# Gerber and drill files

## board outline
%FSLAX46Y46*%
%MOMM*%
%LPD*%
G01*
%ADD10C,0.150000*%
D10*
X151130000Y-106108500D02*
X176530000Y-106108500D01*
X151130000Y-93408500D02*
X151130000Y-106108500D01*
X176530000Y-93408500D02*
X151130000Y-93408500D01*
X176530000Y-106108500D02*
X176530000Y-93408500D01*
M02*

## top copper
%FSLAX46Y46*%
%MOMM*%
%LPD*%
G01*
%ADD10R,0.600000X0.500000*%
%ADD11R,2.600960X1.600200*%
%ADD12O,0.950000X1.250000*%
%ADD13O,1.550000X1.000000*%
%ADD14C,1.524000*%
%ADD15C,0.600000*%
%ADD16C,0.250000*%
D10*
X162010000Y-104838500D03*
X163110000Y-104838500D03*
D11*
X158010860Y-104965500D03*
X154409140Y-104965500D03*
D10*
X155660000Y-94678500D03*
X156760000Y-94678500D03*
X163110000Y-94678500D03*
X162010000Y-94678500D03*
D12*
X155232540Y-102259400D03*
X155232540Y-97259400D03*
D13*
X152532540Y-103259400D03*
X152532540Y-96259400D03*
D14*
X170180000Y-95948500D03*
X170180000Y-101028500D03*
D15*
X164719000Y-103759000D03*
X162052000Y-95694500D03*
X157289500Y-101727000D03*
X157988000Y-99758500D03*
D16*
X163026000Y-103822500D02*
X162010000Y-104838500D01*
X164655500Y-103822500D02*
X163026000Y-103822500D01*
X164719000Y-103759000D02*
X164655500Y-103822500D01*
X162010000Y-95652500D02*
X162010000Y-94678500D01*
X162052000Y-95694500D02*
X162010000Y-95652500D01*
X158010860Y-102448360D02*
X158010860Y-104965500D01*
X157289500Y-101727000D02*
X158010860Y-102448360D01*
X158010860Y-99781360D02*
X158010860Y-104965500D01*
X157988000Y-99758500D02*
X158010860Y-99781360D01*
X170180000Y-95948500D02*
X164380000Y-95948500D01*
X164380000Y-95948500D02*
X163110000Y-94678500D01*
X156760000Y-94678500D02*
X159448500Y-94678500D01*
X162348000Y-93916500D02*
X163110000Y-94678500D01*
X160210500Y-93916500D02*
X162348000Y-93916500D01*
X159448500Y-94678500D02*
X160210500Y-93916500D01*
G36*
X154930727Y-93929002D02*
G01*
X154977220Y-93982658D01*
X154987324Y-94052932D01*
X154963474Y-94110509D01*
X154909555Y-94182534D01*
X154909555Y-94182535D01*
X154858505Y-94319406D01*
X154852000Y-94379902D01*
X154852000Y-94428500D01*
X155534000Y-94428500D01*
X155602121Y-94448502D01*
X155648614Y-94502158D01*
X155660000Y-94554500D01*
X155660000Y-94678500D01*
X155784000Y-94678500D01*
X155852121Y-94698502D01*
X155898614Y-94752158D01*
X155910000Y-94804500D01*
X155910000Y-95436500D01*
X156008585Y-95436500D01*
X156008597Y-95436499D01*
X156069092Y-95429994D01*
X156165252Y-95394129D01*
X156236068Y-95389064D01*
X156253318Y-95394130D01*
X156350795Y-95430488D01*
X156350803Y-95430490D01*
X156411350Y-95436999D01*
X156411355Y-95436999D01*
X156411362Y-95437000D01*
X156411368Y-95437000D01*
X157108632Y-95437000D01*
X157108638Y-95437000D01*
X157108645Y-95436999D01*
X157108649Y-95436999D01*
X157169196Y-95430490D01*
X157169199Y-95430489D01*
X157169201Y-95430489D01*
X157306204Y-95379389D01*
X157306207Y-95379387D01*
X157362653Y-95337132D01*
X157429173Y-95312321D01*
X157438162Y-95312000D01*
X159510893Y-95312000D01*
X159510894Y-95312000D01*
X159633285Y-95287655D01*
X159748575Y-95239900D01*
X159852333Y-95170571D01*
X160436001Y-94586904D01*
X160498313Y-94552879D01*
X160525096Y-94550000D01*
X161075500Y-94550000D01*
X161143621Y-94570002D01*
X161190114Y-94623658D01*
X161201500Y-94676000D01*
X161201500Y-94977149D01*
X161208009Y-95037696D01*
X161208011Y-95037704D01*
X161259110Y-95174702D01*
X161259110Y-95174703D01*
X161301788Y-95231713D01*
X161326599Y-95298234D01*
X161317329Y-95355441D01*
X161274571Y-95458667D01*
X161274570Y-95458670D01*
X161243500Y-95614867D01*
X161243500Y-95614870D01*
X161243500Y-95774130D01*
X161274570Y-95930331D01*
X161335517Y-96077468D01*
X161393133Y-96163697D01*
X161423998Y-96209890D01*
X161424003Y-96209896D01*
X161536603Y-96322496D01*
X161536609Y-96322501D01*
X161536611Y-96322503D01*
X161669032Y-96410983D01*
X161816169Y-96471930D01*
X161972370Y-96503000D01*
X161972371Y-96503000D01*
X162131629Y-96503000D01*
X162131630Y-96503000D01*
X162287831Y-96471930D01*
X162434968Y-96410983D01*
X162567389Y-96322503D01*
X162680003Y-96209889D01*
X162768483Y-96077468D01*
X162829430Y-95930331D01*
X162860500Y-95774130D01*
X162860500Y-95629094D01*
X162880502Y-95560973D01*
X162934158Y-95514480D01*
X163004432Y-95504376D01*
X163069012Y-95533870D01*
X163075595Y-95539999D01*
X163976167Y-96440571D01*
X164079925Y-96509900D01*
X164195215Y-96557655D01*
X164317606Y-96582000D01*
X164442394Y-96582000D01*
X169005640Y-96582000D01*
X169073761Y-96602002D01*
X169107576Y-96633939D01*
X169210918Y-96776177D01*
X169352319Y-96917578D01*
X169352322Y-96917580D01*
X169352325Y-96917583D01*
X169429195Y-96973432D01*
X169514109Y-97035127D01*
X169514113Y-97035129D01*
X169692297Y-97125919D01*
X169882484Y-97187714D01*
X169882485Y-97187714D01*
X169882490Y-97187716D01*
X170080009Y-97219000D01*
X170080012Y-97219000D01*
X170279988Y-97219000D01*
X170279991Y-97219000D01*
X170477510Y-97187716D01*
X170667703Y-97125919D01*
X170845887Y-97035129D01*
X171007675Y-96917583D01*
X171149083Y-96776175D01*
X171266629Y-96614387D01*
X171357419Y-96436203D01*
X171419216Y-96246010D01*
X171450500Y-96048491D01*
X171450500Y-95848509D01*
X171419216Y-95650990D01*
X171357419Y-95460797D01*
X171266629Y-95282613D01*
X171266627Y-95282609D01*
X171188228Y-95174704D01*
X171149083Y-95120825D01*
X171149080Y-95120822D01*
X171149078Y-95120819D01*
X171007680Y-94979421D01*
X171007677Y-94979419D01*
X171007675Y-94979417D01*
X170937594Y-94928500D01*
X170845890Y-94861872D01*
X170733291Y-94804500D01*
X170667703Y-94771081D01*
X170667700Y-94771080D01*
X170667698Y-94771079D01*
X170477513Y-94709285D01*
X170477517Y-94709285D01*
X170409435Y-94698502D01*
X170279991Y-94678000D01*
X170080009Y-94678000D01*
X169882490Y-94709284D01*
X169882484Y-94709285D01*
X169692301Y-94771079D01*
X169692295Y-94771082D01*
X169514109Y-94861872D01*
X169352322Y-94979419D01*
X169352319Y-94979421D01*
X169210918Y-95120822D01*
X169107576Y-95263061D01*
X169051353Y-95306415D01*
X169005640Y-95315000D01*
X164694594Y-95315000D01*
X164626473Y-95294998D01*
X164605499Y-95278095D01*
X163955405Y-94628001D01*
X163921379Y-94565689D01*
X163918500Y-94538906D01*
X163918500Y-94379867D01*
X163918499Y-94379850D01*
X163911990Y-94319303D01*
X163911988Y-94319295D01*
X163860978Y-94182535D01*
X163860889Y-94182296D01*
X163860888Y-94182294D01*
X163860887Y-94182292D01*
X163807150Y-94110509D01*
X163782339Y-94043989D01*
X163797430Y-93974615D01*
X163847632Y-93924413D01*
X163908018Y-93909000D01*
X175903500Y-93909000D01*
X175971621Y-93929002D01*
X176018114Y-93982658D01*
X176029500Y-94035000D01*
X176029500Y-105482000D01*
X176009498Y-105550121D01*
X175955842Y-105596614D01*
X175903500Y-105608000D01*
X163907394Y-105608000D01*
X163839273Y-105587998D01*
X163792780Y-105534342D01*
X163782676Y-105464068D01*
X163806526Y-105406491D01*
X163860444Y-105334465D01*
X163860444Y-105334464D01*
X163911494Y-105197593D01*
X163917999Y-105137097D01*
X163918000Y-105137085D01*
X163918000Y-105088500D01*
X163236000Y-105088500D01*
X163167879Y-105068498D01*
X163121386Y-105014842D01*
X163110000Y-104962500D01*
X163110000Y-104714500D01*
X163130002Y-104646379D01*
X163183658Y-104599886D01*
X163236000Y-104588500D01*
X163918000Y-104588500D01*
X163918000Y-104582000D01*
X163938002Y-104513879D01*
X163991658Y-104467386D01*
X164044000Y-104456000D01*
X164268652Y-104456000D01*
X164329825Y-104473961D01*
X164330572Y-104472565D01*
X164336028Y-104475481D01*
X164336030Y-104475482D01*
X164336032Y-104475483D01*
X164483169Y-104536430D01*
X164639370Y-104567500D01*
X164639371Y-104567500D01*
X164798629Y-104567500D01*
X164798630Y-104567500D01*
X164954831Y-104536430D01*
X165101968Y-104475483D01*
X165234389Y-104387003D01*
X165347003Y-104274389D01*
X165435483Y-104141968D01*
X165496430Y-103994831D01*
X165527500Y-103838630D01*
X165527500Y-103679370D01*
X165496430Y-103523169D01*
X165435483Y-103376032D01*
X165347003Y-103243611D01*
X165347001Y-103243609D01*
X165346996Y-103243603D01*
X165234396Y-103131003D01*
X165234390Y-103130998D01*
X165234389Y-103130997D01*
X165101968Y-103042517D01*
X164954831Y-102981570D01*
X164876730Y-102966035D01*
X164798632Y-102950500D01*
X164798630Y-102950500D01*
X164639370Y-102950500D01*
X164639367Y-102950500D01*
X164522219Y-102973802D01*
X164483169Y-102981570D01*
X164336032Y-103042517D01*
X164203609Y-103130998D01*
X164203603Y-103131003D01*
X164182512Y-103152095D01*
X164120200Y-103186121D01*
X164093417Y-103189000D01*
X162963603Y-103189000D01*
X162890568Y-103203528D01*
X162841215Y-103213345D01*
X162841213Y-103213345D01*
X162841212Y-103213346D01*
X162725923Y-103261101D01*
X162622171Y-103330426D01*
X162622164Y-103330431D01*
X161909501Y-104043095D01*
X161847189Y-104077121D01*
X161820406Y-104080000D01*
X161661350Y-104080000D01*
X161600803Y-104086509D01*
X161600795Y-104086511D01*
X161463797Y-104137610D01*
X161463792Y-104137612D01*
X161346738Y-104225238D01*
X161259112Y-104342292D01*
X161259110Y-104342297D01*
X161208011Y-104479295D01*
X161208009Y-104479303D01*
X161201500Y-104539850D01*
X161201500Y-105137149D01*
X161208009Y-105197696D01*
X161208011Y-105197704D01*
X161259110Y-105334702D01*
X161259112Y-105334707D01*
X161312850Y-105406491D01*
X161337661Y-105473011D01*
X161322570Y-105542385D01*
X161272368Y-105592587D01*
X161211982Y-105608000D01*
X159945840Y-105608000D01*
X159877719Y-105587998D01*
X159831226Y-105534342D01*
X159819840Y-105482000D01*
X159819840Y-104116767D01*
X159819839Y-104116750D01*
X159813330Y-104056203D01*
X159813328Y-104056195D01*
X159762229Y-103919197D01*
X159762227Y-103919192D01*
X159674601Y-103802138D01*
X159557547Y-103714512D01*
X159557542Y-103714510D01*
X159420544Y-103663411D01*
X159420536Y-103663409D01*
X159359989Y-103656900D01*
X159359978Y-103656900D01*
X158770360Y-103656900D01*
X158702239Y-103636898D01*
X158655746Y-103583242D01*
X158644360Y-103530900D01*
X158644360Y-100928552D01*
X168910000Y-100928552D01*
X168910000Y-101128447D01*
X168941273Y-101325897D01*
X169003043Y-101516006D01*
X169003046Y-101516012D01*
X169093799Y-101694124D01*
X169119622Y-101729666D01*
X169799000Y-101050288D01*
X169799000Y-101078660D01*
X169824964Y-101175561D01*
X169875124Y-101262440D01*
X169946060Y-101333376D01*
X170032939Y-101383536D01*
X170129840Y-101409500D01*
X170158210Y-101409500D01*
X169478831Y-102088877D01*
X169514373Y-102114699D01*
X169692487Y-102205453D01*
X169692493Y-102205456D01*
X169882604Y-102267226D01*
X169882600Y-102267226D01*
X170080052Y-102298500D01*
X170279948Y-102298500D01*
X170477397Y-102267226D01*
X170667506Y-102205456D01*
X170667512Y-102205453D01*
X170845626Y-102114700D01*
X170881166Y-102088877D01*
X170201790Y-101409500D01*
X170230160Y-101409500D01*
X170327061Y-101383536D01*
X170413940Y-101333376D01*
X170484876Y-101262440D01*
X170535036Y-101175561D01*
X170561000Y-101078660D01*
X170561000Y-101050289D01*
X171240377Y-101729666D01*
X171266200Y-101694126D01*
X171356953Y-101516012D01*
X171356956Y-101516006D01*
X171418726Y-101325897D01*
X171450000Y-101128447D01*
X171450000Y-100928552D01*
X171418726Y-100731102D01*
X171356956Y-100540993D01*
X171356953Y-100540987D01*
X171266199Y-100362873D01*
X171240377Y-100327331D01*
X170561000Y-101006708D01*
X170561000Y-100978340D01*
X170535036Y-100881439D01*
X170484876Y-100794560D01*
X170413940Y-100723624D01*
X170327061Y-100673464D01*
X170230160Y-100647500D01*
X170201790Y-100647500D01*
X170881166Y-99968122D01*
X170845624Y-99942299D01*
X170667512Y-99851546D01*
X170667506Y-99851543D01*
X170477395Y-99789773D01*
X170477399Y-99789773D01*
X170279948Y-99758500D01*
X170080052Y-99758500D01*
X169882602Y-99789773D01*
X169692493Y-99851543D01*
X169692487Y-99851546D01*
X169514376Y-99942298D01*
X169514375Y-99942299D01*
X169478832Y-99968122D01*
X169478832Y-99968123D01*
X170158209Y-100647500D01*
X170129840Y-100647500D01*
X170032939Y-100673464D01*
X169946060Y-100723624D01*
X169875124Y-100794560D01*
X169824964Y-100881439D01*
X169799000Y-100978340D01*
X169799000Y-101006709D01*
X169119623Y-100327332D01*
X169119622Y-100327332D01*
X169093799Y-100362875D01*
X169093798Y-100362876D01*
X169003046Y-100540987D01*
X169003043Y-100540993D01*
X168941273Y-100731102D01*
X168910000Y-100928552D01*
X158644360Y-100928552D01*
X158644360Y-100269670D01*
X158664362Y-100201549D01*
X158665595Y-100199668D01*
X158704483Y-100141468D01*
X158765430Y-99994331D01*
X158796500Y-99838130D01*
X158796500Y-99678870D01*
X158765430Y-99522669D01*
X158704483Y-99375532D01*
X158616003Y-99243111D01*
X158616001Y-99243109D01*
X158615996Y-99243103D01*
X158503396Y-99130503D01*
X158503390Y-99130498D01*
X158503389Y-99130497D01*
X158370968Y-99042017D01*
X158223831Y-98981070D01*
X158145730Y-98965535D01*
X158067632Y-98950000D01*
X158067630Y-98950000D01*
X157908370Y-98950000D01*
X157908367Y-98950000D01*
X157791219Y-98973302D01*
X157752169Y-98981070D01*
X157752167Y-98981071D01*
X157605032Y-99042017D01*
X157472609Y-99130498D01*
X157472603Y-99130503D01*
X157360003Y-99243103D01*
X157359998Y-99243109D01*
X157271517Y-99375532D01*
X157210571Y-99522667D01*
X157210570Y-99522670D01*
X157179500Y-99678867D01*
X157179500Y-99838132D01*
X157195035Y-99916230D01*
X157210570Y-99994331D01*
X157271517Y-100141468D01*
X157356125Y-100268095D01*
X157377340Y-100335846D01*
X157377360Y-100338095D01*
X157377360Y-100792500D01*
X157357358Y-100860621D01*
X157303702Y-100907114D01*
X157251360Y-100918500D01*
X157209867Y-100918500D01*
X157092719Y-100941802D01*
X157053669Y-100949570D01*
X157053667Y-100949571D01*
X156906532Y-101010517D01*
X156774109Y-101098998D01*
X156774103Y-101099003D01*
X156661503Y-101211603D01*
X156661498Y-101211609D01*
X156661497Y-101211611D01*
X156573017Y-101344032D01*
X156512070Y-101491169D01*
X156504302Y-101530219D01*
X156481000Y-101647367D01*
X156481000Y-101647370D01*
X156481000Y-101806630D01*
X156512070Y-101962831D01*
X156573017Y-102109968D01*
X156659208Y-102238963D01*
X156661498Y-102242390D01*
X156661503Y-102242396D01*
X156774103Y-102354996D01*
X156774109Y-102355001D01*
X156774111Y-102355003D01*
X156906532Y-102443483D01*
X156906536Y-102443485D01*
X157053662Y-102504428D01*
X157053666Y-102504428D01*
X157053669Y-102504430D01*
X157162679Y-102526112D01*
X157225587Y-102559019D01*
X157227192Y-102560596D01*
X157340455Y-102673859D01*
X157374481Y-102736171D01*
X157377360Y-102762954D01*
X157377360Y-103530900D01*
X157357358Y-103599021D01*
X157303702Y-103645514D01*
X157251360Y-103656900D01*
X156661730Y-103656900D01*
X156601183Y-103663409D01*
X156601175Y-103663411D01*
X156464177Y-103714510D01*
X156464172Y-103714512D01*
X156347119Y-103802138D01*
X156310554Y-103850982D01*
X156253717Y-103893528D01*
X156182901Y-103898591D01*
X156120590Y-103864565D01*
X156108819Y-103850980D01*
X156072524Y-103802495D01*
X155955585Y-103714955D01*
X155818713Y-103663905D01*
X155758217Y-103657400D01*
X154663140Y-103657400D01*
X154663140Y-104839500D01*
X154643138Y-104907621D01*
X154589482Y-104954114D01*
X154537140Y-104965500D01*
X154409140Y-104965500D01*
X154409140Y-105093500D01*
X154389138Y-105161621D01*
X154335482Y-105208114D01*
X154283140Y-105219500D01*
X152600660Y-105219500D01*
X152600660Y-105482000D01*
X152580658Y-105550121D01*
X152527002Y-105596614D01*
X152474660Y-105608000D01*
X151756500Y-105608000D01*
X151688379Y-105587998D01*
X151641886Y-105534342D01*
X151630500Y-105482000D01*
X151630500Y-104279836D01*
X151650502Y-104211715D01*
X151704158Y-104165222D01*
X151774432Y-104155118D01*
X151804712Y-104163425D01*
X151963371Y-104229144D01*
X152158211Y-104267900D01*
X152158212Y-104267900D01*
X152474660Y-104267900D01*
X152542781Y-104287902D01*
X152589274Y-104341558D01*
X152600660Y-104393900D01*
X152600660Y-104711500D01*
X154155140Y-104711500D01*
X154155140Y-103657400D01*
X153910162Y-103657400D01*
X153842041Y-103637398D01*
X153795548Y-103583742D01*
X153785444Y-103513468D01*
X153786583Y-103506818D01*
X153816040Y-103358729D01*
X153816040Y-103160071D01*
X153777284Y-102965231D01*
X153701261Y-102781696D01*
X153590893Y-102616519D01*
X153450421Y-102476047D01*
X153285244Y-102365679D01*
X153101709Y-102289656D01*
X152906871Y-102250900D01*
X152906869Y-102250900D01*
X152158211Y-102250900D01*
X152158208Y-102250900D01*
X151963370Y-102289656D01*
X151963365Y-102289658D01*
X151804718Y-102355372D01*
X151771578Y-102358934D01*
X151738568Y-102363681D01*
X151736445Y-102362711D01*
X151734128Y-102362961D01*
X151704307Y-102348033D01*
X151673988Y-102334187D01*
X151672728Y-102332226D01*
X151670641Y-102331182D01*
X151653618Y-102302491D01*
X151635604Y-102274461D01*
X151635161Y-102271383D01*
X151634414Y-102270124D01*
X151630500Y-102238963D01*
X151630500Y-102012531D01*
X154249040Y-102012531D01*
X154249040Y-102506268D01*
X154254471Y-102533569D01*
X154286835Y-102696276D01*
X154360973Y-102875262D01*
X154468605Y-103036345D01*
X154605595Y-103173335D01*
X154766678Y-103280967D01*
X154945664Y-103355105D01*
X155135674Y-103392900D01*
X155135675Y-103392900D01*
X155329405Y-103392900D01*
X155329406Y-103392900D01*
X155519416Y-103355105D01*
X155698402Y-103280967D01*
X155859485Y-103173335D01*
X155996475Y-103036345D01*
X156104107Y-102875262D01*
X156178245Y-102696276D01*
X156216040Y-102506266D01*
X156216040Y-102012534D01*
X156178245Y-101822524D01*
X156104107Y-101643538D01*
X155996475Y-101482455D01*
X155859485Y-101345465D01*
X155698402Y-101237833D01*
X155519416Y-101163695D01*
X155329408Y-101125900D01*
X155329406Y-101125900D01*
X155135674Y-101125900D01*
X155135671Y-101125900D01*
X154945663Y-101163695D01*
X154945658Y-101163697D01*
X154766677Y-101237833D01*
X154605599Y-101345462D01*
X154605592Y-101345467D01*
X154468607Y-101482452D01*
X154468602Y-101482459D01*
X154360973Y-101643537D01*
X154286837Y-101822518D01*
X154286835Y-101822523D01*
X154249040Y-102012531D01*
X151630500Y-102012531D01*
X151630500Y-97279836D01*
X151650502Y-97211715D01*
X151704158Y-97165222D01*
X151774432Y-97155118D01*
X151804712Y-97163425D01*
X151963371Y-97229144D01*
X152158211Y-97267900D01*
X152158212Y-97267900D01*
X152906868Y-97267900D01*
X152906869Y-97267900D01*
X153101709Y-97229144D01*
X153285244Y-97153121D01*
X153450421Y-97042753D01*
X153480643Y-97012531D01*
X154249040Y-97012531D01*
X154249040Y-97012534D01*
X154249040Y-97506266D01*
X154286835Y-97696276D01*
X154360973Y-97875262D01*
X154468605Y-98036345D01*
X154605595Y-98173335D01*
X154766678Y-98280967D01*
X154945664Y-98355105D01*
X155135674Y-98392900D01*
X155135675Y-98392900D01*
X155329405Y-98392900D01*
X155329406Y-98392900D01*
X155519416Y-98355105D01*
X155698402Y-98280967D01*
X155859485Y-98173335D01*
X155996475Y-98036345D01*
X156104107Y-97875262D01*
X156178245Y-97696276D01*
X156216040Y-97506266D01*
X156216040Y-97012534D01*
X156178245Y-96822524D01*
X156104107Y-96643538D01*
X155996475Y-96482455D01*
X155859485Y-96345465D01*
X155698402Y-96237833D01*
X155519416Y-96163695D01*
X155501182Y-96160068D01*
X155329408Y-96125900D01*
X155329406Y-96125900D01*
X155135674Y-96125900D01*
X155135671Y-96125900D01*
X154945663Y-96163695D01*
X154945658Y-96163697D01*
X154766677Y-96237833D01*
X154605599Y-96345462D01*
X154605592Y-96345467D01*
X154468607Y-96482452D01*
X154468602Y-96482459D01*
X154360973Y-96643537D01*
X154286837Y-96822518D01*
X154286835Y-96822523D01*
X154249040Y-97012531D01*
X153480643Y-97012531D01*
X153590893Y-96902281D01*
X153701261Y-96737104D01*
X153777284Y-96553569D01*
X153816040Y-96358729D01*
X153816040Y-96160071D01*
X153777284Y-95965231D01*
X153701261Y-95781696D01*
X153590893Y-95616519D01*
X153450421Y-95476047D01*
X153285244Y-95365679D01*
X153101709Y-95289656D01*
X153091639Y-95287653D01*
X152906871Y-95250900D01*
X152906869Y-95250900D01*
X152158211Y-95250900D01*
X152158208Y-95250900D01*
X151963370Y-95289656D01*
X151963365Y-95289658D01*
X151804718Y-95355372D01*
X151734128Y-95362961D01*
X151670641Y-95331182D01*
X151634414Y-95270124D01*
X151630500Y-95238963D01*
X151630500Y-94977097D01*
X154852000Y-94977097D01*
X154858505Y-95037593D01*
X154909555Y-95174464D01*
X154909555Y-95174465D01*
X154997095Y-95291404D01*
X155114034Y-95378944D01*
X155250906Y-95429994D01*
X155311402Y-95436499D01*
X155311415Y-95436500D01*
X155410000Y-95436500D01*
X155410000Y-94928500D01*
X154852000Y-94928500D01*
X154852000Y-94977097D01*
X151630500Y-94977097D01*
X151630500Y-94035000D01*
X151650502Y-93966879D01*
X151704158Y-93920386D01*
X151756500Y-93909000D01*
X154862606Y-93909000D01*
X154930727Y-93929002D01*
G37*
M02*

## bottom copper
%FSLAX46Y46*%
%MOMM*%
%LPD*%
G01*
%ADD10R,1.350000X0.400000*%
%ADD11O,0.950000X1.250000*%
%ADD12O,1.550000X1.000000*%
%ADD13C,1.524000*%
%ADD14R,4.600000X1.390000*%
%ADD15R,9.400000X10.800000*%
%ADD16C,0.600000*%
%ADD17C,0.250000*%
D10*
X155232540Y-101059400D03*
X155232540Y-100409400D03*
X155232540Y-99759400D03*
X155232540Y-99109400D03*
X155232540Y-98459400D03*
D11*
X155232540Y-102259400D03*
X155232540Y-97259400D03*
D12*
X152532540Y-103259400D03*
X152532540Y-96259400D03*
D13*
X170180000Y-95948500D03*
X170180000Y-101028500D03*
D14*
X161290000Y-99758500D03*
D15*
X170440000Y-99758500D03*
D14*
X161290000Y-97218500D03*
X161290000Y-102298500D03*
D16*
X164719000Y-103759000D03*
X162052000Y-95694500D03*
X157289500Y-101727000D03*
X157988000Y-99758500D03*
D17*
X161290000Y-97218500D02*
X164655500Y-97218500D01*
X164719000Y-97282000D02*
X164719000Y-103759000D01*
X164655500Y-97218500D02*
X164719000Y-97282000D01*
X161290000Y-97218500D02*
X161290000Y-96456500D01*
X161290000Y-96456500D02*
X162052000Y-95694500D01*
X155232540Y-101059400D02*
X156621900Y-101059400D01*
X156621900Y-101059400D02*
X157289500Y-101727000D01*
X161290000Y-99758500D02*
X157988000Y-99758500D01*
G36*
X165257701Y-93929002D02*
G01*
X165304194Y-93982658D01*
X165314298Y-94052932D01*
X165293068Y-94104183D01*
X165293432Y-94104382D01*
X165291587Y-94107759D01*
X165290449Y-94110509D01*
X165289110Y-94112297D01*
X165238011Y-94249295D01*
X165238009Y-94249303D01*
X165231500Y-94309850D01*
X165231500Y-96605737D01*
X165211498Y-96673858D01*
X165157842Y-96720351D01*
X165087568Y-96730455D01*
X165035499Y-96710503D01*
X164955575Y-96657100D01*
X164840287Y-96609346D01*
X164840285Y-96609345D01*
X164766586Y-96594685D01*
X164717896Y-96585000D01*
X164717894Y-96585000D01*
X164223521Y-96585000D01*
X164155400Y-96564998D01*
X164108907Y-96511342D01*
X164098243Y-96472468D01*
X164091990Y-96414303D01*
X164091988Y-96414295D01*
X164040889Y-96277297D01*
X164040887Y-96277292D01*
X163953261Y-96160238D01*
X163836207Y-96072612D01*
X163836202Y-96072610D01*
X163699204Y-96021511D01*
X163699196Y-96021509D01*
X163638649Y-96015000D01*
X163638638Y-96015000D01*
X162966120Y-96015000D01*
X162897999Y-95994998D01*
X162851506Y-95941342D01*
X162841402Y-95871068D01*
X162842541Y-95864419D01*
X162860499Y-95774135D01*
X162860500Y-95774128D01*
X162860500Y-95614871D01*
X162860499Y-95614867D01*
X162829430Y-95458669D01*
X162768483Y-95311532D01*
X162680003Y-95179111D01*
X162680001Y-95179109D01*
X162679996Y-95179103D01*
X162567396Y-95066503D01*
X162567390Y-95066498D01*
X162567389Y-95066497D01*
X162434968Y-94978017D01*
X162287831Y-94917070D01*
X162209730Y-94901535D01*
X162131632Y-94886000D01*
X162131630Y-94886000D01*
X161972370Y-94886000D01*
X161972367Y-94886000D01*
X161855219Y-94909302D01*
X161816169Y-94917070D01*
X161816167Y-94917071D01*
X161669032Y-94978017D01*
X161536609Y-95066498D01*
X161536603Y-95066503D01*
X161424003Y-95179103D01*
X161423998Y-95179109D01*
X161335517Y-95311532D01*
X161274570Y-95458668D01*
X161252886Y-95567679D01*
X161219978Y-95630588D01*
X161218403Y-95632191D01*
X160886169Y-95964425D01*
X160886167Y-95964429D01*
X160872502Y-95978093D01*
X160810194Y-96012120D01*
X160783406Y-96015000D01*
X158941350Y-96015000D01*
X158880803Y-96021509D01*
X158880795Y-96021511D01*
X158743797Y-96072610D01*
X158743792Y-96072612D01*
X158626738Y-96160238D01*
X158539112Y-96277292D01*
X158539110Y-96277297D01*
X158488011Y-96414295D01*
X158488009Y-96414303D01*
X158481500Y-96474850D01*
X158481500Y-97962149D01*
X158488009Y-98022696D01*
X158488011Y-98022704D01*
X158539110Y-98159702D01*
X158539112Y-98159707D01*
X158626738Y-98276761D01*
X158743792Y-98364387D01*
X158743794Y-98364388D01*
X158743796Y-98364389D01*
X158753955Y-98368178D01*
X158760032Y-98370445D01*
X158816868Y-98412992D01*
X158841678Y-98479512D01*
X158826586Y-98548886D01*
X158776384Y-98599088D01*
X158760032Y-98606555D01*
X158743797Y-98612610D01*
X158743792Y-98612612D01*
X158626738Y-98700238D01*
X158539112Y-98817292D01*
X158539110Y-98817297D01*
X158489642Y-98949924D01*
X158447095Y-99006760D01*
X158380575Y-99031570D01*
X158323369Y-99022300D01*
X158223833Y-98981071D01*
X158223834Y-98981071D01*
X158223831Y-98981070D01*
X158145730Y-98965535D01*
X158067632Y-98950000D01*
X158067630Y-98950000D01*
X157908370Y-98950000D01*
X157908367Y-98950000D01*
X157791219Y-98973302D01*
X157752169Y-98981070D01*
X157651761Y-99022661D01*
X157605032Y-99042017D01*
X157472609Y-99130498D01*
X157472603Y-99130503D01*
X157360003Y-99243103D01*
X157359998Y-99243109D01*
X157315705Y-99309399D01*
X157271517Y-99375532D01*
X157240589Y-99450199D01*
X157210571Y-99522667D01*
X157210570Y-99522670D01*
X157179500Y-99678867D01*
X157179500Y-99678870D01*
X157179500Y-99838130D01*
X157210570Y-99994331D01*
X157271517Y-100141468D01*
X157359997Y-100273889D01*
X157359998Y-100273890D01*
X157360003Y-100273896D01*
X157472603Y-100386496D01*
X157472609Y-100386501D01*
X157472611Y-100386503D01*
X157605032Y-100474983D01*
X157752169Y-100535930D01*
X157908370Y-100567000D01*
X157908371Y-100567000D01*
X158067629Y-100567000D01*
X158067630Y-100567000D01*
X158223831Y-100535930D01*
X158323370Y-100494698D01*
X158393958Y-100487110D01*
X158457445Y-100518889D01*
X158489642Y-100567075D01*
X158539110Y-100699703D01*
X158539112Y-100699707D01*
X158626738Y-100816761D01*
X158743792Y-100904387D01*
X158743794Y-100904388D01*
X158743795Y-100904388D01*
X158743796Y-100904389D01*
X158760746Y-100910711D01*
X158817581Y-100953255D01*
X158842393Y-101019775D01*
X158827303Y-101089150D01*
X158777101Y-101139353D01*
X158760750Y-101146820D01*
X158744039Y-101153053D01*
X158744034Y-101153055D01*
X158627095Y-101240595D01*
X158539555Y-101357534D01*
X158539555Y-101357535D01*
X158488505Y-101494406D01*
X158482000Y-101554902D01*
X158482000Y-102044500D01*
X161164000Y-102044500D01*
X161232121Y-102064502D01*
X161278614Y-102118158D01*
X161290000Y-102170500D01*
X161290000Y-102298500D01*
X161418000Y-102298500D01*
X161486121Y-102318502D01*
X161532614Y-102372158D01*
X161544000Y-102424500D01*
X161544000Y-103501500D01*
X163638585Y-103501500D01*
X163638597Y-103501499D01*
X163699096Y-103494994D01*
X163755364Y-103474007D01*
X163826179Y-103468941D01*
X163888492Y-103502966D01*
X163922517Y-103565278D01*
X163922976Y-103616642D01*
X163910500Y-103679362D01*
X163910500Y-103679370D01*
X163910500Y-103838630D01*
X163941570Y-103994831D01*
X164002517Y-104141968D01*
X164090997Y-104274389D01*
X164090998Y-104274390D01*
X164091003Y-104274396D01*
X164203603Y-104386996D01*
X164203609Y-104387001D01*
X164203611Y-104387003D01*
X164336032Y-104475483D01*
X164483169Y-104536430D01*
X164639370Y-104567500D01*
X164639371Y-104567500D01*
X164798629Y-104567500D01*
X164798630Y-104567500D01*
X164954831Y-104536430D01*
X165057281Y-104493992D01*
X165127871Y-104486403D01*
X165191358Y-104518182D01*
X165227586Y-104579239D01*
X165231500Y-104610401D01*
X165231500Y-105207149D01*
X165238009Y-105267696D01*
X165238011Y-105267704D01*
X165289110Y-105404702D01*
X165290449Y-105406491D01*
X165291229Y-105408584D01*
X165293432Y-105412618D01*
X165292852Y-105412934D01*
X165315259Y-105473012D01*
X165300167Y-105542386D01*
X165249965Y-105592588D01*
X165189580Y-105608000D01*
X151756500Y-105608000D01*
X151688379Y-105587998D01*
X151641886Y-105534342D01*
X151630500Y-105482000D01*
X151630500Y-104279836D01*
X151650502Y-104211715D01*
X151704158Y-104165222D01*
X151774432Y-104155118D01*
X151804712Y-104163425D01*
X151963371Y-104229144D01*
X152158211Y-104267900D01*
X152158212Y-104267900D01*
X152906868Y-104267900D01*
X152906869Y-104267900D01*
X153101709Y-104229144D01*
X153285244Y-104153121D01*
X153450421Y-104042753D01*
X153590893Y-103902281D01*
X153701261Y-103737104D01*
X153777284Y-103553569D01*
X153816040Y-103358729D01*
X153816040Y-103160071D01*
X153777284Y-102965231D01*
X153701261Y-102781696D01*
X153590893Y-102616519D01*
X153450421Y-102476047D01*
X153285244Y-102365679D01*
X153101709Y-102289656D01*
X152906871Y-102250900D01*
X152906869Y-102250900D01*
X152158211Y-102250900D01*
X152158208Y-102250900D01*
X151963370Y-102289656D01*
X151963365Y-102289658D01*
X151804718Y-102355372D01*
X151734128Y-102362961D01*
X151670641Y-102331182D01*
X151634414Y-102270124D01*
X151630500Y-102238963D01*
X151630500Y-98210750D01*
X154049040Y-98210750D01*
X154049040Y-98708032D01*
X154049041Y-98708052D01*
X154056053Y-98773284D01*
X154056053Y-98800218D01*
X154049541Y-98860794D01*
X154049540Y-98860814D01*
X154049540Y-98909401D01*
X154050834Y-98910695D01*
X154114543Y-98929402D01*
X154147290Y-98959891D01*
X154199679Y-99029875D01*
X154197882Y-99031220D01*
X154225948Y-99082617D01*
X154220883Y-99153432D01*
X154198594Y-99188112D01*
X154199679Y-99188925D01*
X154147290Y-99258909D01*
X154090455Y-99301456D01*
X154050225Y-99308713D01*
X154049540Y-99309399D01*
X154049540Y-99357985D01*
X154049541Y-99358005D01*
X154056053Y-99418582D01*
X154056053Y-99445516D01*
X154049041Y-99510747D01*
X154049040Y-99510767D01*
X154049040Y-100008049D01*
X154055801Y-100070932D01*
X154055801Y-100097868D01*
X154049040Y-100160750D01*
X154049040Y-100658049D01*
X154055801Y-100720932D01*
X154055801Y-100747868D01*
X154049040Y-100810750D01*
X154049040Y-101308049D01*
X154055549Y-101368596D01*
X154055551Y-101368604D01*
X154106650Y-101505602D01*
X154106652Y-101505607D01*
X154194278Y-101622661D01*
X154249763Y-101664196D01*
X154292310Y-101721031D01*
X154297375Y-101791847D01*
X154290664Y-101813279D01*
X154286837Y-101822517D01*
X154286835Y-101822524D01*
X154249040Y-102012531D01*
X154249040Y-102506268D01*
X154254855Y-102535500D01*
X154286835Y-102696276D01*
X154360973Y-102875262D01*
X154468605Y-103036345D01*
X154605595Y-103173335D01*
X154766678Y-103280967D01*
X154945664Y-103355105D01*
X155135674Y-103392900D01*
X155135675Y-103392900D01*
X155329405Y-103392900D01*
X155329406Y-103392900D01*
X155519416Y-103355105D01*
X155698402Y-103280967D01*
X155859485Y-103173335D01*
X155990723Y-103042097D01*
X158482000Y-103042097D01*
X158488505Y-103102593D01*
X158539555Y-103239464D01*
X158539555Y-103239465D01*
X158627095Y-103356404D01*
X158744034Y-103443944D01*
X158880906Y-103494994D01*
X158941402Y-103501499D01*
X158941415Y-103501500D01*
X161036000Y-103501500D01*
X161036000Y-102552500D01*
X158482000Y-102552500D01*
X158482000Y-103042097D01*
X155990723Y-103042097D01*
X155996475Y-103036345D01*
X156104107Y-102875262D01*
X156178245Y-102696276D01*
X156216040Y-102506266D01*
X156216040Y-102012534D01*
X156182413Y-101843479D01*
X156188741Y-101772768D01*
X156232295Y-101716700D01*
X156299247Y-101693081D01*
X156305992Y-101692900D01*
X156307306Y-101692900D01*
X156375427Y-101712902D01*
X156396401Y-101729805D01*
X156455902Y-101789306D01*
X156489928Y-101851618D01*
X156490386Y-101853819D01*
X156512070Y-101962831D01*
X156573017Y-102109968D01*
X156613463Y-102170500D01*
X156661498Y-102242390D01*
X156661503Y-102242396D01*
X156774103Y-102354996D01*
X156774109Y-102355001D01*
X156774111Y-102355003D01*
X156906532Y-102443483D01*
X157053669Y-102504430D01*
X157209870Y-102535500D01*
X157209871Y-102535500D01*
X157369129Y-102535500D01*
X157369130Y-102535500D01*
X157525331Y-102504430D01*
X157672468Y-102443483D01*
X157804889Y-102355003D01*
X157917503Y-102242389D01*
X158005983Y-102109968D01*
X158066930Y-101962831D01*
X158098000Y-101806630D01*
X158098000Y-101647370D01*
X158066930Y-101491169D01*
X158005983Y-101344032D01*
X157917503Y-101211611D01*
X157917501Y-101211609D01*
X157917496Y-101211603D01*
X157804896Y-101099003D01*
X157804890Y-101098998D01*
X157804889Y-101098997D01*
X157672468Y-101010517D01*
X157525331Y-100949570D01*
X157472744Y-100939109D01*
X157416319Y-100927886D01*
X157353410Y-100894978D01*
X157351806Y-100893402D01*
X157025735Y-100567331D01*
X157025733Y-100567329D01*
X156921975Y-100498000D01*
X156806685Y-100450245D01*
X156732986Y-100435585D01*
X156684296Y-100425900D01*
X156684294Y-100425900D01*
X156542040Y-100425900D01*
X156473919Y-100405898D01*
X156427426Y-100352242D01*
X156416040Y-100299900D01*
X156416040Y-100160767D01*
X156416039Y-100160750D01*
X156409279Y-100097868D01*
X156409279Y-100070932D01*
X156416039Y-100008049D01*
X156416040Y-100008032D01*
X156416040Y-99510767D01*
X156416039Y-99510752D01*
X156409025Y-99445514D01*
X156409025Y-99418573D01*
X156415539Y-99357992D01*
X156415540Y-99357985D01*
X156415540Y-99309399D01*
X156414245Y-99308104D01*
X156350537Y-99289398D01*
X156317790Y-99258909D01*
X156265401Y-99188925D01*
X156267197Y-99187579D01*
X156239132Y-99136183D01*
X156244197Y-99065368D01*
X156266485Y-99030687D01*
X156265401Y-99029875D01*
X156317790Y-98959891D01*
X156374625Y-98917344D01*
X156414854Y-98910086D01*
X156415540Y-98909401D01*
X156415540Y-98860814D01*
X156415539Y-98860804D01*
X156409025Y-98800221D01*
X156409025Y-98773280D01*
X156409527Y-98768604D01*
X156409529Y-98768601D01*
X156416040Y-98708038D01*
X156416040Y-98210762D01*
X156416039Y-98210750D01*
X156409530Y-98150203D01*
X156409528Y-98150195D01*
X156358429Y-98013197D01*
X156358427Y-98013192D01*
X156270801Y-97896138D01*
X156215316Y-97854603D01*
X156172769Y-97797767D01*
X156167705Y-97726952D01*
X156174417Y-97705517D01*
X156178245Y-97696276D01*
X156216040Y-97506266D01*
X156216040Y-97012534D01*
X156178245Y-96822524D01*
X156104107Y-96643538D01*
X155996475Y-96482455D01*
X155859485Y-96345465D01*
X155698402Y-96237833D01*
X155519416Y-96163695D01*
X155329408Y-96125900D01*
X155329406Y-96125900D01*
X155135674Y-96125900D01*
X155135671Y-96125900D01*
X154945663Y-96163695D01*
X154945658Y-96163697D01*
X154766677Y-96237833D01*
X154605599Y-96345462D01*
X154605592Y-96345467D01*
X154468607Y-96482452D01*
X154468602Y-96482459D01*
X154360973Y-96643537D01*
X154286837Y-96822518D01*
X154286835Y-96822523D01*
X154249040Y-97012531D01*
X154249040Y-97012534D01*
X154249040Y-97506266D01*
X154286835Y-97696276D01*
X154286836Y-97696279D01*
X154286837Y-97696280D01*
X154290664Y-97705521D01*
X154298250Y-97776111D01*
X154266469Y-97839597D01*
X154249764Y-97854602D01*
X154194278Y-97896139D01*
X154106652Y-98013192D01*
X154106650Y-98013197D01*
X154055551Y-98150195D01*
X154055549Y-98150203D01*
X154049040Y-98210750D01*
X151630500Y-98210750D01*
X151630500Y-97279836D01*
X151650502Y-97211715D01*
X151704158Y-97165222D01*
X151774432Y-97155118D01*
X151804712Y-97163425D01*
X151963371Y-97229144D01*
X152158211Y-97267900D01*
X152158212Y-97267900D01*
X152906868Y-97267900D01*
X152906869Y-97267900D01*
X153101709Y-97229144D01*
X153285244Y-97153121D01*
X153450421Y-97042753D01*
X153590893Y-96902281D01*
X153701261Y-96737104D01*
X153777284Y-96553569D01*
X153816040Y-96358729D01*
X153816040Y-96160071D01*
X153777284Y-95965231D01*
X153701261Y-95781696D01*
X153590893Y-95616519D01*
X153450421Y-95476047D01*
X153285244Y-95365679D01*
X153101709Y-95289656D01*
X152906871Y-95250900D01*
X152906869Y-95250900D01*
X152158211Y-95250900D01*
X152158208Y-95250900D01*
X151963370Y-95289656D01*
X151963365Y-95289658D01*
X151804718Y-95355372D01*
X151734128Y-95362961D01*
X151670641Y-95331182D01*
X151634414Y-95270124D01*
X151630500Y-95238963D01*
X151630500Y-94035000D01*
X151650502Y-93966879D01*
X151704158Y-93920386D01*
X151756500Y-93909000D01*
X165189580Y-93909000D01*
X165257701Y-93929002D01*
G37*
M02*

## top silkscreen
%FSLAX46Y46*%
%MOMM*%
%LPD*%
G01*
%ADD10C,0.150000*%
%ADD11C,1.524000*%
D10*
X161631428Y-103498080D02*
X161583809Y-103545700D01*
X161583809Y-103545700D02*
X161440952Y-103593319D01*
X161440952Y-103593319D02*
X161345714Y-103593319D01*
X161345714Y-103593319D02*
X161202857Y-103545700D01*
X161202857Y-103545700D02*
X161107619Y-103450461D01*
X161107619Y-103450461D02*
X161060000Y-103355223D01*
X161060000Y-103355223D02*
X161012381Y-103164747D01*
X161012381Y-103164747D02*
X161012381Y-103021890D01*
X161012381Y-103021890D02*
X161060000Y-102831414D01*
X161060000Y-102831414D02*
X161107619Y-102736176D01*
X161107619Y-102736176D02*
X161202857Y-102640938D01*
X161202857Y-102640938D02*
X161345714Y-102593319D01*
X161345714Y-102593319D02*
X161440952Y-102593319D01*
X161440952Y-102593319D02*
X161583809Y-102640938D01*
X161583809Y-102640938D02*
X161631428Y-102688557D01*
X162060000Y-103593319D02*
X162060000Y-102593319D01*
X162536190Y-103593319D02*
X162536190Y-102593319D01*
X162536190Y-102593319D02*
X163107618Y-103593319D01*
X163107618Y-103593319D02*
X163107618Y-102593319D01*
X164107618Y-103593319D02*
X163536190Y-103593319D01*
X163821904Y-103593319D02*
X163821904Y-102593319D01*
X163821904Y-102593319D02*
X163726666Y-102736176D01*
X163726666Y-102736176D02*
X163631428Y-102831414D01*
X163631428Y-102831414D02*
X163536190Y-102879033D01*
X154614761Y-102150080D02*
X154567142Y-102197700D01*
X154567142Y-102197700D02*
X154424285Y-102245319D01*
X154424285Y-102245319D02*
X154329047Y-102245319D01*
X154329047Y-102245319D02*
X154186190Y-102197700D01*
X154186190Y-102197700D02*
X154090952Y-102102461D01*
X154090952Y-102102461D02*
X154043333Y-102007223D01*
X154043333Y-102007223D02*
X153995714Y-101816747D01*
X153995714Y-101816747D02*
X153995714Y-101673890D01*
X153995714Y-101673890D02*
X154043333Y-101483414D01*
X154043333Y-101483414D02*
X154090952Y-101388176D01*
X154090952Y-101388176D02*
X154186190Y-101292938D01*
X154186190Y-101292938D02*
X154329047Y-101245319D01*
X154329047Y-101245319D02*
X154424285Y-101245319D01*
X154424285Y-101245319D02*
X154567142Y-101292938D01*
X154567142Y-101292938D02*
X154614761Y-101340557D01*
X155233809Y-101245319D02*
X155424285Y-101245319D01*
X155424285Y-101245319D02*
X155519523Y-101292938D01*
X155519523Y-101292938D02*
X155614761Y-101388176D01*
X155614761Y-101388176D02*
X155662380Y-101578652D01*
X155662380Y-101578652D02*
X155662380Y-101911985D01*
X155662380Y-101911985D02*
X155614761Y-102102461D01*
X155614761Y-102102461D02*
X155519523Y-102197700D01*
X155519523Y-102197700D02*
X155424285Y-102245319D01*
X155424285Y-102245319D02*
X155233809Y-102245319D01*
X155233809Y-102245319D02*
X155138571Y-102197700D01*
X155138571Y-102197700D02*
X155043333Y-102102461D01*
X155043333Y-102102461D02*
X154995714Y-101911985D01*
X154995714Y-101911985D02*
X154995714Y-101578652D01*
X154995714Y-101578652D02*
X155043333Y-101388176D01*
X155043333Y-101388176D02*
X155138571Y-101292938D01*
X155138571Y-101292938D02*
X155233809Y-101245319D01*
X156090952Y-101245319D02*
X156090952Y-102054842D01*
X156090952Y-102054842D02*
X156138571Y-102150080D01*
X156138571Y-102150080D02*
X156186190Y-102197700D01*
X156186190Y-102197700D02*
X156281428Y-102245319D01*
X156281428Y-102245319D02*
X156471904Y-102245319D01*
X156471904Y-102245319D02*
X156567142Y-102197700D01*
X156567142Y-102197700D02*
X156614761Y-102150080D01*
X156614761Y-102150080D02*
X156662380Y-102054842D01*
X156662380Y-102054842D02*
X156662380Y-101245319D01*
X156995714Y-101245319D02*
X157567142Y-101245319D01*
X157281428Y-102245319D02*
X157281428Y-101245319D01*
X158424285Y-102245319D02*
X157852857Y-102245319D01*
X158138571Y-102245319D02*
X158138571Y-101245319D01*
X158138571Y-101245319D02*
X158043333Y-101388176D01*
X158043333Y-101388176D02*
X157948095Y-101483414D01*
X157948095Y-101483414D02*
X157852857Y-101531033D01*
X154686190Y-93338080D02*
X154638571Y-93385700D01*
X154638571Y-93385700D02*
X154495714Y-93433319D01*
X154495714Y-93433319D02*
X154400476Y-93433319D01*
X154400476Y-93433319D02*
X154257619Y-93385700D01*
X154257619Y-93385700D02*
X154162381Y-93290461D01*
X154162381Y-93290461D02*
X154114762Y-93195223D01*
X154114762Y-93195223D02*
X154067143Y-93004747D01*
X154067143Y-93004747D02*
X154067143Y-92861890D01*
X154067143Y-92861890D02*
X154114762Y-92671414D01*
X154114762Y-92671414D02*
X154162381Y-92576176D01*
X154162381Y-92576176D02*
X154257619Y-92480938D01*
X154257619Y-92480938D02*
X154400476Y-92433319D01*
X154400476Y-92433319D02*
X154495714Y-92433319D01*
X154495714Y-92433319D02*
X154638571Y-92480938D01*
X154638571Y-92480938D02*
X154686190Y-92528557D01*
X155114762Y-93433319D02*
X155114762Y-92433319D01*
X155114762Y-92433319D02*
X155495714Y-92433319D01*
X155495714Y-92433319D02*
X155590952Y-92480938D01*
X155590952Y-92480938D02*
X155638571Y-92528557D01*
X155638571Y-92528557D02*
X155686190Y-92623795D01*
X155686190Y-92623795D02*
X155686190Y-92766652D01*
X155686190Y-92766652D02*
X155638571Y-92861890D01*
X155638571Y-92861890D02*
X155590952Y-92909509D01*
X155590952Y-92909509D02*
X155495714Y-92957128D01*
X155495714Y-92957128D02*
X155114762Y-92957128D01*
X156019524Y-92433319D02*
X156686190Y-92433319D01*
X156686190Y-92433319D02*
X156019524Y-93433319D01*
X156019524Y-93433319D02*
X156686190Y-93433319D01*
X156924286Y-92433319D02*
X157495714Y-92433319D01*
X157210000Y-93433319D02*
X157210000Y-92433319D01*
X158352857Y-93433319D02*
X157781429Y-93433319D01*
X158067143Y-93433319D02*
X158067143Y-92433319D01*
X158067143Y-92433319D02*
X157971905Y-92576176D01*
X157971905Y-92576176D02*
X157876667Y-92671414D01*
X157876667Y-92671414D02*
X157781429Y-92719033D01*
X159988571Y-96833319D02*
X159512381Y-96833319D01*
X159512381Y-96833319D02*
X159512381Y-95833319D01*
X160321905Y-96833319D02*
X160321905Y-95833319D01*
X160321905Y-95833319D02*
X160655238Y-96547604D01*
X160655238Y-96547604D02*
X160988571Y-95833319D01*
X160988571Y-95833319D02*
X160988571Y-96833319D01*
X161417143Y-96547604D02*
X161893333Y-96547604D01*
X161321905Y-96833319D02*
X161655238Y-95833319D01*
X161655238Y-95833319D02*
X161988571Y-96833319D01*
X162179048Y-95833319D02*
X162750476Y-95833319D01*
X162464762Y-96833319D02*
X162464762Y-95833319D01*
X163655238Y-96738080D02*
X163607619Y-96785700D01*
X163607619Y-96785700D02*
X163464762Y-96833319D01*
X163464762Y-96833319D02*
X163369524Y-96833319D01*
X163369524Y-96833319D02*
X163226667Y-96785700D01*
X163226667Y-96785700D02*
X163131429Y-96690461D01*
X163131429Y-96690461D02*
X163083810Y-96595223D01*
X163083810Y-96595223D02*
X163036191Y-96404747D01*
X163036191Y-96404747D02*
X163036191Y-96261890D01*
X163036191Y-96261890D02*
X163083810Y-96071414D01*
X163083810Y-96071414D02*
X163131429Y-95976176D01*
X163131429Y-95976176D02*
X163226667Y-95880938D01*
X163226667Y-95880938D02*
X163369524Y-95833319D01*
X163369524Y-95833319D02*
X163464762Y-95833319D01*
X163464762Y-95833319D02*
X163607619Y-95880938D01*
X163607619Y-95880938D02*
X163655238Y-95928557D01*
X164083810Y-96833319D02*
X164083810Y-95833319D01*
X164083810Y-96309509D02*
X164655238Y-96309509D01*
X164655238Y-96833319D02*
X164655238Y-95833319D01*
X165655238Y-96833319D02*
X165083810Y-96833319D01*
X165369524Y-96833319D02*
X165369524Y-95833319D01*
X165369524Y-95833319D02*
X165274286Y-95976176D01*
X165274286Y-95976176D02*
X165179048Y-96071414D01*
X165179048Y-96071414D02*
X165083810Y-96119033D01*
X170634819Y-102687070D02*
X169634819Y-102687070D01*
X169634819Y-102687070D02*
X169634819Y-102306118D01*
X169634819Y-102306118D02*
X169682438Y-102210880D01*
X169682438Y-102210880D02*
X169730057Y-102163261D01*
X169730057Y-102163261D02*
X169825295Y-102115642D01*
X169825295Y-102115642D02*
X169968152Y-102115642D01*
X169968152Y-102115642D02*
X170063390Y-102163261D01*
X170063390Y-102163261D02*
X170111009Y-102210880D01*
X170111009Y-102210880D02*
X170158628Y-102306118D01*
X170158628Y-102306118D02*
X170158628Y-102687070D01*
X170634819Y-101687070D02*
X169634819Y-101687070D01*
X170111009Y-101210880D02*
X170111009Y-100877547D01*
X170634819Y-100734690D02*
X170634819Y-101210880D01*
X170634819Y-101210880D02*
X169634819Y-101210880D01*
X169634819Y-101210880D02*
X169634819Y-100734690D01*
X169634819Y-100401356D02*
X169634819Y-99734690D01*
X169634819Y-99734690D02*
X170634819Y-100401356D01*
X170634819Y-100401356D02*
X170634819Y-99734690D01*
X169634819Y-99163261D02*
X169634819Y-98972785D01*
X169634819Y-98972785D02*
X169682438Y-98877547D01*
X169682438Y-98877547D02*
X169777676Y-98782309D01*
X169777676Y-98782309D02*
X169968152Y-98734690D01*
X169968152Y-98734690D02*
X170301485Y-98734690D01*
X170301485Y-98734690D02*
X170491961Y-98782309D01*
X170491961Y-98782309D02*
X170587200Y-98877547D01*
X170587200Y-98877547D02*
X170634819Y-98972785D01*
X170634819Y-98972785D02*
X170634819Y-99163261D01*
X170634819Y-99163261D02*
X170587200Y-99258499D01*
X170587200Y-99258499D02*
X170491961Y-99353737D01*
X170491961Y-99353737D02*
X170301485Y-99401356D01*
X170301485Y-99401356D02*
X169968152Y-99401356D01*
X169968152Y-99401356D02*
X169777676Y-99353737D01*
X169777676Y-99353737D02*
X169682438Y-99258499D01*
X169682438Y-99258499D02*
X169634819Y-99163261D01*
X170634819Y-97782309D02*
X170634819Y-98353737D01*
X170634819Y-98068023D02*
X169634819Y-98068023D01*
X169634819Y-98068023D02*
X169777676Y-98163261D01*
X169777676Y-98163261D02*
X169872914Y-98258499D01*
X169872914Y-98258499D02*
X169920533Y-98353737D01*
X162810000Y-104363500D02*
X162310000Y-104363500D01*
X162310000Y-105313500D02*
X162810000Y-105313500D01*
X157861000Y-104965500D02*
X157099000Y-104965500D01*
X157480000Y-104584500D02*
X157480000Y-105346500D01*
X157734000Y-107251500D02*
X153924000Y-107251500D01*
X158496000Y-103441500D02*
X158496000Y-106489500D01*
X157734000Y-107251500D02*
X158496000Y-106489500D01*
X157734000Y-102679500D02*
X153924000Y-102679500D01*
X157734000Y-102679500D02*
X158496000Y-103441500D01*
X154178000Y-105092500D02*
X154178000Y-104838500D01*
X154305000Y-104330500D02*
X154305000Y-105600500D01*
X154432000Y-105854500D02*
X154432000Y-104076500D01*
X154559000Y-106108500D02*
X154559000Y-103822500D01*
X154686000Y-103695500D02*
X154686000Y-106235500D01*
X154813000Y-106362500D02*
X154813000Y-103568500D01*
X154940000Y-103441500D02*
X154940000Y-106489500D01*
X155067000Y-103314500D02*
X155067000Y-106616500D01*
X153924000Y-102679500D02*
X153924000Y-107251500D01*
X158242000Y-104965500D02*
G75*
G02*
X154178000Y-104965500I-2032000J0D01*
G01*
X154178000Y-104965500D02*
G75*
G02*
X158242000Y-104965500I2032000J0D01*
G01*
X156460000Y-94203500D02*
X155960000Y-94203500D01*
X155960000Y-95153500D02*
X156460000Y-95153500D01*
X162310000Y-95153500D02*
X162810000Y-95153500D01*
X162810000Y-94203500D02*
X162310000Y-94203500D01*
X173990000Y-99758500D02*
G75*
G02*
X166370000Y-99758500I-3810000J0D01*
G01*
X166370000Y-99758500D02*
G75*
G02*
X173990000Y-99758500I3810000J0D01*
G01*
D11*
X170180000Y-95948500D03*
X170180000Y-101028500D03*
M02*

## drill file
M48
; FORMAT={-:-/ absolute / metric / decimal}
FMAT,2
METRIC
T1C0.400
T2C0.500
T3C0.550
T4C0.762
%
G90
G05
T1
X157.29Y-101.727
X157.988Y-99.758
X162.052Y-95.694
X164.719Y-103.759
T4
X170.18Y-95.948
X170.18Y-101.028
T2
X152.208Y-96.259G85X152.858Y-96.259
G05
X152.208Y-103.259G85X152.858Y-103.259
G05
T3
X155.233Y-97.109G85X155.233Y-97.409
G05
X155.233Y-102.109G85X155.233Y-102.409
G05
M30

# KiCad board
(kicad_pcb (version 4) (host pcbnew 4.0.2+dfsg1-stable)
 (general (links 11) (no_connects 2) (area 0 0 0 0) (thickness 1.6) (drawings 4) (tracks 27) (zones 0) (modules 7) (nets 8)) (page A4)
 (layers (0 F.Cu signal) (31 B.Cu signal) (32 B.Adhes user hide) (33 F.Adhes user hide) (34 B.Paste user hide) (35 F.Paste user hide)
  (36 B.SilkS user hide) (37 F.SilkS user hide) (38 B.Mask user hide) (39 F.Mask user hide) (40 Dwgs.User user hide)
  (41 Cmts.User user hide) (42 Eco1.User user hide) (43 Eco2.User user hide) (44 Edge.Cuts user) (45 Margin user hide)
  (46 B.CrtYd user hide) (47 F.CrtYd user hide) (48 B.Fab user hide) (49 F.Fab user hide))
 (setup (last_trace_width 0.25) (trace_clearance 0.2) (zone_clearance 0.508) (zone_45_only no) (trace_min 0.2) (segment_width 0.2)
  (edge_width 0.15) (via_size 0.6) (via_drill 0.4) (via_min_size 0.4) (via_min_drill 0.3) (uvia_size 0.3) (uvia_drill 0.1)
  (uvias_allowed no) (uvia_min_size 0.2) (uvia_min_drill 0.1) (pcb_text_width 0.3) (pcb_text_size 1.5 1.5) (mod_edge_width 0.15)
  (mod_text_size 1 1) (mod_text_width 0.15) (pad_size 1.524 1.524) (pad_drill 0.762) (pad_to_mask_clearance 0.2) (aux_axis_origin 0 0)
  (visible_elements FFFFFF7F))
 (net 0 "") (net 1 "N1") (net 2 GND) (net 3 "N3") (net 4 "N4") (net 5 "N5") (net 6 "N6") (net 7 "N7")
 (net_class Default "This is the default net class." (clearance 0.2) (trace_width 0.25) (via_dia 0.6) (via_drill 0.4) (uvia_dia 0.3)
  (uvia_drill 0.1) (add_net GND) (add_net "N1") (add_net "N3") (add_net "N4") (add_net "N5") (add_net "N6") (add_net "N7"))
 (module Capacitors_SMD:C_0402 (layer F.Cu) (at 162.56 104.8385)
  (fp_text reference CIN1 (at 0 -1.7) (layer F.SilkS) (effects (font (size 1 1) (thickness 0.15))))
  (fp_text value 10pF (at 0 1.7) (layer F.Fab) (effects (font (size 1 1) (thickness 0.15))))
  (fp_line (start 0.25 -0.475) (end -0.25 -0.475) (layer F.SilkS) (width 0.15))
  (fp_line (start -0.25 0.475) (end 0.25 0.475) (layer F.SilkS) (width 0.15))
  (pad 1 smd rect (at -0.55 0) (size 0.6 0.5) (layers F.Cu F.Paste F.Mask) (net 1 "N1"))
  (pad 2 smd rect (at 0.55 0) (size 0.6 0.5) (layers F.Cu F.Paste F.Mask) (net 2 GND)))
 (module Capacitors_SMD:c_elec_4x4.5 (layer F.Cu) (at 156.21 104.9655)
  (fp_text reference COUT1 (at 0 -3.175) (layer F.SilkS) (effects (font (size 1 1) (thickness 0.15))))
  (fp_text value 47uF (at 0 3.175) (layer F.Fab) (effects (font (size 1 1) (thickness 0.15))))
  (fp_line (start 1.651 0) (end 0.889 0) (layer F.SilkS) (width 0.15))
  (fp_line (start 1.27 -0.381) (end 1.27 0.381) (layer F.SilkS) (width 0.15))
  (fp_line (start 1.524 2.286) (end -2.286 2.286) (layer F.SilkS) (width 0.15))
  (fp_line (start 2.286 -1.524) (end 2.286 1.524) (layer F.SilkS) (width 0.15))
  (fp_line (start 1.524 2.286) (end 2.286 1.524) (layer F.SilkS) (width 0.15))
  (fp_line (start 1.524 -2.286) (end -2.286 -2.286) (layer F.SilkS) (width 0.15))
  (fp_line (start 1.524 -2.286) (end 2.286 -1.524) (layer F.SilkS) (width 0.15))
  (fp_line (start -2.032 0.127) (end -2.032 -0.127) (layer F.SilkS) (width 0.15))
  (fp_line (start -1.905 -0.635) (end -1.905 0.635) (layer F.SilkS) (width 0.15))
  (fp_line (start -1.778 0.889) (end -1.778 -0.889) (layer F.SilkS) (width 0.15))
  (fp_line (start -1.651 1.143) (end -1.651 -1.143) (layer F.SilkS) (width 0.15))
  (fp_line (start -1.524 -1.27) (end -1.524 1.27) (layer F.SilkS) (width 0.15))
  (fp_line (start -1.397 1.397) (end -1.397 -1.397) (layer F.SilkS) (width 0.15))
  (fp_line (start -1.27 -1.524) (end -1.27 1.524) (layer F.SilkS) (width 0.15))
  (fp_line (start -1.143 -1.651) (end -1.143 1.651) (layer F.SilkS) (width 0.15))
  (fp_line (start -2.286 -2.286) (end -2.286 2.286) (layer F.SilkS) (width 0.15))
  (fp_circle (center 0 0) (end -2.032 0) (layer F.SilkS) (width 0.15))
  (pad 1 smd rect (at 1.80086 0) (size 2.60096 1.6002) (layers F.Cu F.Paste F.Mask) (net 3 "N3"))
  (pad 2 smd rect (at -1.80086 0) (size 2.60096 1.6002) (layers F.Cu F.Paste F.Mask) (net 2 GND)))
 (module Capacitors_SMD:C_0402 (layer F.Cu) (at 156.21 94.6785)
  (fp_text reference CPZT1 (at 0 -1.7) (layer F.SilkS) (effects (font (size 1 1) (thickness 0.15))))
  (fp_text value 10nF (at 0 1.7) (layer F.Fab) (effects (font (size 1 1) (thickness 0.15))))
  (fp_line (start 0.25 -0.475) (end -0.25 -0.475) (layer F.SilkS) (width 0.15))
  (fp_line (start -0.25 0.475) (end 0.25 0.475) (layer F.SilkS) (width 0.15))
  (pad 1 smd rect (at -0.55 0) (size 0.6 0.5) (layers F.Cu F.Paste F.Mask) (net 2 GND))
  (pad 2 smd rect (at 0.55 0) (size 0.6 0.5) (layers F.Cu F.Paste F.Mask) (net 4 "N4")))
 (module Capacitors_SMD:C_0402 (layer F.Cu) (at 162.56 94.6785 180)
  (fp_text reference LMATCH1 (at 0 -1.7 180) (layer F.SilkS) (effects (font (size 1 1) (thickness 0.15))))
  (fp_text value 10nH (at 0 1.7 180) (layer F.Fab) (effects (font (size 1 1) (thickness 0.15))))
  (fp_line (start 0.25 -0.475) (end -0.25 -0.475) (layer F.SilkS) (width 0.15))
  (fp_line (start -0.25 0.475) (end 0.25 0.475) (layer F.SilkS) (width 0.15))
  (pad 1 smd rect (at -0.55 0 180) (size 0.6 0.5) (layers F.Cu F.Paste F.Mask) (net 4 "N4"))
  (pad 2 smd rect (at 0.55 0 180) (size 0.6 0.5) (layers F.Cu F.Paste F.Mask) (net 1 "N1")))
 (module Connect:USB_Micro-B (layer B.Cu) (at 153.67 99.7585 90)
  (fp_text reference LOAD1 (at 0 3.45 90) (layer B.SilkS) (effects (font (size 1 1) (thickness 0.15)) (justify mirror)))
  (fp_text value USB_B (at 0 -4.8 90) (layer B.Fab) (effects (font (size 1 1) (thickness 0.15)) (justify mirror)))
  (pad 1 smd rect (at -1.3009 1.56254) (size 1.35 0.4) (layers B.Cu B.Paste B.Mask) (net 3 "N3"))
  (pad 2 smd rect (at -0.6509 1.56254) (size 1.35 0.4) (layers B.Cu B.Paste B.Mask) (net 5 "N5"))
  (pad 3 smd rect (at -0.0009 1.56254) (size 1.35 0.4) (layers B.Cu B.Paste B.Mask) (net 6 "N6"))
  (pad 4 smd rect (at 0.6491 1.56254) (size 1.35 0.4) (layers B.Cu B.Paste B.Mask) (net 2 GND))
  (pad 5 smd rect (at 1.2991 1.56254) (size 1.35 0.4) (layers B.Cu B.Paste B.Mask) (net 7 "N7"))
  (pad 6 thru_hole oval (at -2.5009 1.56254) (size 0.95 1.25) (drill oval 0.55 0.85) (layers *.Cu *.Mask B.SilkS))
  (pad 6 thru_hole oval (at 2.4991 1.56254) (size 0.95 1.25) (drill oval 0.55 0.85) (layers *.Cu *.Mask B.SilkS))
  (pad 6 thru_hole oval (at -3.5009 -1.13746) (size 1.55 1) (drill oval 1.15 0.5) (layers *.Cu *.Mask B.SilkS))
  (pad 6 thru_hole oval (at 3.4991 -1.13746) (size 1.55 1) (drill oval 1.15 0.5) (layers *.Cu *.Mask B.SilkS)))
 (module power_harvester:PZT (layer F.Cu) (at 170.18 99.7585)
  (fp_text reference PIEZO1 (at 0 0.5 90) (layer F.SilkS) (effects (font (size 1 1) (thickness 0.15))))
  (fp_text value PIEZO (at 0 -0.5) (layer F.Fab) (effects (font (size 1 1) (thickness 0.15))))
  (fp_circle (center 0 0) (end 3.81 0) (layer F.SilkS) (width 0.15))
  (pad 1 thru_hole circle (at 0 -3.81) (size 1.524 1.524) (drill 0.762) (layers *.Cu *.Mask F.SilkS) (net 4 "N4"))
  (pad 2 thru_hole circle (at 0 1.27) (size 1.524 1.524) (drill 0.762) (layers *.Cu *.Mask F.SilkS) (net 2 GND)))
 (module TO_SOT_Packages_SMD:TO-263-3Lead (layer B.Cu) (at 161.29 99.7585)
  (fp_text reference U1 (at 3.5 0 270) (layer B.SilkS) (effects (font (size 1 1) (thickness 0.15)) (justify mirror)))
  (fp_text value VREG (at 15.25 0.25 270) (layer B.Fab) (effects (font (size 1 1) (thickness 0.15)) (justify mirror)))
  (pad 2 smd rect (at 0 0) (size 4.6 1.39) (layers B.Cu B.Paste B.Mask) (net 3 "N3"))
  (pad 4 smd rect (at 9.15 0) (size 9.4 10.8) (layers B.Cu B.Paste B.Mask))
  (pad 3 smd rect (at 0 -2.54) (size 4.6 1.39) (layers B.Cu B.Paste B.Mask) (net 1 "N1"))
  (pad 1 smd rect (at 0 2.54) (size 4.6 1.39) (layers B.Cu B.Paste B.Mask) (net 2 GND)))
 (gr_line (start 151.13 106.1085) (end 176.53 106.1085) (angle 90) (layer Edge.Cuts) (width 0.15))
 (gr_line (start 151.13 93.4085) (end 151.13 106.1085) (angle 90) (layer Edge.Cuts) (width 0.15))
 (gr_line (start 176.53 93.4085) (end 151.13 93.4085) (angle 90) (layer Edge.Cuts) (width 0.15))
 (gr_line (start 176.53 106.1085) (end 176.53 93.4085) (angle 90) (layer Edge.Cuts) (width 0.15))
 (segment (start 161.29 97.2185) (end 164.6555 97.2185) (width 0.25) (layer B.Cu) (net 1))
 (segment (start 163.026 103.8225) (end 162.01 104.8385) (width 0.25) (layer F.Cu) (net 1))
 (segment (start 164.6555 103.8225) (end 163.026 103.8225) (width 0.25) (layer F.Cu) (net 1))
 (segment (start 164.719 103.759) (end 164.6555 103.8225) (width 0.25) (layer F.Cu) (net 1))
 (via (at 164.719 103.759) (size 0.6) (drill 0.4) (layers F.Cu B.Cu) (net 1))
 (segment (start 164.719 97.282) (end 164.719 103.759) (width 0.25) (layer B.Cu) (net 1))
 (segment (start 164.6555 97.2185) (end 164.719 97.282) (width 0.25) (layer B.Cu) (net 1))
 (segment (start 161.29 97.2185) (end 161.29 96.4565) (width 0.25) (layer B.Cu) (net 1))
 (segment (start 162.01 95.6525) (end 162.01 94.6785) (width 0.25) (layer F.Cu) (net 1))
 (segment (start 162.052 95.6945) (end 162.01 95.6525) (width 0.25) (layer F.Cu) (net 1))
 (via (at 162.052 95.6945) (size 0.6) (drill 0.4) (layers F.Cu B.Cu) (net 1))
 (segment (start 161.29 96.4565) (end 162.052 95.6945) (width 0.25) (layer B.Cu) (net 1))
 (segment (start 155.23254 101.0594) (end 156.6219 101.0594) (width 0.25) (layer B.Cu) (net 3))
 (segment (start 158.01086 102.44836) (end 158.01086 104.9655) (width 0.25) (layer F.Cu) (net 3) (status 20))
 (segment (start 157.2895 101.727) (end 158.01086 102.44836) (width 0.25) (layer F.Cu) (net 3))
 (via (at 157.2895 101.727) (size 0.6) (drill 0.4) (layers F.Cu B.Cu) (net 3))
 (segment (start 156.6219 101.0594) (end 157.2895 101.727) (width 0.25) (layer B.Cu) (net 3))
 (segment (start 161.29 99.7585) (end 157.988 99.7585) (width 0.25) (layer B.Cu) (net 3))
 (segment (start 158.01086 99.78136) (end 158.01086 104.9655) (width 0.25) (layer F.Cu) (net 3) (status 20))
 (segment (start 157.988 99.7585) (end 158.01086 99.78136) (width 0.25) (layer F.Cu) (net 3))
 (via (at 157.988 99.7585) (size 0.6) (drill 0.4) (layers F.Cu B.Cu) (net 3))
 (segment (start 170.18 95.9485) (end 164.38 95.9485) (width 0.25) (layer F.Cu) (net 4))
 (segment (start 164.38 95.9485) (end 163.11 94.6785) (width 0.25) (layer F.Cu) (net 4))
 (segment (start 156.76 94.6785) (end 159.4485 94.6785) (width 0.25) (layer F.Cu) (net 4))
 (segment (start 162.348 93.9165) (end 163.11 94.6785) (width 0.25) (layer F.Cu) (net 4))
 (segment (start 160.2105 93.9165) (end 162.348 93.9165) (width 0.25) (layer F.Cu) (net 4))
 (segment (start 159.4485 94.6785) (end 160.2105 93.9165) (width 0.25) (layer F.Cu) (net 4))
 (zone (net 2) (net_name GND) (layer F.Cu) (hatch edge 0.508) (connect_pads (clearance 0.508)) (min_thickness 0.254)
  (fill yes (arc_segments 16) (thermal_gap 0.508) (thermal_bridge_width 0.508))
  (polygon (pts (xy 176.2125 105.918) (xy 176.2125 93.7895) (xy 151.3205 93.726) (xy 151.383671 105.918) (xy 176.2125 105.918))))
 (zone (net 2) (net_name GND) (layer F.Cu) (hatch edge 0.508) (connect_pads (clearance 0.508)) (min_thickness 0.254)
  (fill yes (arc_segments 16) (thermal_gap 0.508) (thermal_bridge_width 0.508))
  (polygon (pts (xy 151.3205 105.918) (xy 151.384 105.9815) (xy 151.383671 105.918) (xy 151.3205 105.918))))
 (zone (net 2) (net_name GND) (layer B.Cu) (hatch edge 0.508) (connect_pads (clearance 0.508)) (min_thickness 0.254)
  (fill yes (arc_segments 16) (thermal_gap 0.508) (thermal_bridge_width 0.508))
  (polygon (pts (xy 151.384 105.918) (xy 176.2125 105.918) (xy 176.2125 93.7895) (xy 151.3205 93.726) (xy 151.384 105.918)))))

